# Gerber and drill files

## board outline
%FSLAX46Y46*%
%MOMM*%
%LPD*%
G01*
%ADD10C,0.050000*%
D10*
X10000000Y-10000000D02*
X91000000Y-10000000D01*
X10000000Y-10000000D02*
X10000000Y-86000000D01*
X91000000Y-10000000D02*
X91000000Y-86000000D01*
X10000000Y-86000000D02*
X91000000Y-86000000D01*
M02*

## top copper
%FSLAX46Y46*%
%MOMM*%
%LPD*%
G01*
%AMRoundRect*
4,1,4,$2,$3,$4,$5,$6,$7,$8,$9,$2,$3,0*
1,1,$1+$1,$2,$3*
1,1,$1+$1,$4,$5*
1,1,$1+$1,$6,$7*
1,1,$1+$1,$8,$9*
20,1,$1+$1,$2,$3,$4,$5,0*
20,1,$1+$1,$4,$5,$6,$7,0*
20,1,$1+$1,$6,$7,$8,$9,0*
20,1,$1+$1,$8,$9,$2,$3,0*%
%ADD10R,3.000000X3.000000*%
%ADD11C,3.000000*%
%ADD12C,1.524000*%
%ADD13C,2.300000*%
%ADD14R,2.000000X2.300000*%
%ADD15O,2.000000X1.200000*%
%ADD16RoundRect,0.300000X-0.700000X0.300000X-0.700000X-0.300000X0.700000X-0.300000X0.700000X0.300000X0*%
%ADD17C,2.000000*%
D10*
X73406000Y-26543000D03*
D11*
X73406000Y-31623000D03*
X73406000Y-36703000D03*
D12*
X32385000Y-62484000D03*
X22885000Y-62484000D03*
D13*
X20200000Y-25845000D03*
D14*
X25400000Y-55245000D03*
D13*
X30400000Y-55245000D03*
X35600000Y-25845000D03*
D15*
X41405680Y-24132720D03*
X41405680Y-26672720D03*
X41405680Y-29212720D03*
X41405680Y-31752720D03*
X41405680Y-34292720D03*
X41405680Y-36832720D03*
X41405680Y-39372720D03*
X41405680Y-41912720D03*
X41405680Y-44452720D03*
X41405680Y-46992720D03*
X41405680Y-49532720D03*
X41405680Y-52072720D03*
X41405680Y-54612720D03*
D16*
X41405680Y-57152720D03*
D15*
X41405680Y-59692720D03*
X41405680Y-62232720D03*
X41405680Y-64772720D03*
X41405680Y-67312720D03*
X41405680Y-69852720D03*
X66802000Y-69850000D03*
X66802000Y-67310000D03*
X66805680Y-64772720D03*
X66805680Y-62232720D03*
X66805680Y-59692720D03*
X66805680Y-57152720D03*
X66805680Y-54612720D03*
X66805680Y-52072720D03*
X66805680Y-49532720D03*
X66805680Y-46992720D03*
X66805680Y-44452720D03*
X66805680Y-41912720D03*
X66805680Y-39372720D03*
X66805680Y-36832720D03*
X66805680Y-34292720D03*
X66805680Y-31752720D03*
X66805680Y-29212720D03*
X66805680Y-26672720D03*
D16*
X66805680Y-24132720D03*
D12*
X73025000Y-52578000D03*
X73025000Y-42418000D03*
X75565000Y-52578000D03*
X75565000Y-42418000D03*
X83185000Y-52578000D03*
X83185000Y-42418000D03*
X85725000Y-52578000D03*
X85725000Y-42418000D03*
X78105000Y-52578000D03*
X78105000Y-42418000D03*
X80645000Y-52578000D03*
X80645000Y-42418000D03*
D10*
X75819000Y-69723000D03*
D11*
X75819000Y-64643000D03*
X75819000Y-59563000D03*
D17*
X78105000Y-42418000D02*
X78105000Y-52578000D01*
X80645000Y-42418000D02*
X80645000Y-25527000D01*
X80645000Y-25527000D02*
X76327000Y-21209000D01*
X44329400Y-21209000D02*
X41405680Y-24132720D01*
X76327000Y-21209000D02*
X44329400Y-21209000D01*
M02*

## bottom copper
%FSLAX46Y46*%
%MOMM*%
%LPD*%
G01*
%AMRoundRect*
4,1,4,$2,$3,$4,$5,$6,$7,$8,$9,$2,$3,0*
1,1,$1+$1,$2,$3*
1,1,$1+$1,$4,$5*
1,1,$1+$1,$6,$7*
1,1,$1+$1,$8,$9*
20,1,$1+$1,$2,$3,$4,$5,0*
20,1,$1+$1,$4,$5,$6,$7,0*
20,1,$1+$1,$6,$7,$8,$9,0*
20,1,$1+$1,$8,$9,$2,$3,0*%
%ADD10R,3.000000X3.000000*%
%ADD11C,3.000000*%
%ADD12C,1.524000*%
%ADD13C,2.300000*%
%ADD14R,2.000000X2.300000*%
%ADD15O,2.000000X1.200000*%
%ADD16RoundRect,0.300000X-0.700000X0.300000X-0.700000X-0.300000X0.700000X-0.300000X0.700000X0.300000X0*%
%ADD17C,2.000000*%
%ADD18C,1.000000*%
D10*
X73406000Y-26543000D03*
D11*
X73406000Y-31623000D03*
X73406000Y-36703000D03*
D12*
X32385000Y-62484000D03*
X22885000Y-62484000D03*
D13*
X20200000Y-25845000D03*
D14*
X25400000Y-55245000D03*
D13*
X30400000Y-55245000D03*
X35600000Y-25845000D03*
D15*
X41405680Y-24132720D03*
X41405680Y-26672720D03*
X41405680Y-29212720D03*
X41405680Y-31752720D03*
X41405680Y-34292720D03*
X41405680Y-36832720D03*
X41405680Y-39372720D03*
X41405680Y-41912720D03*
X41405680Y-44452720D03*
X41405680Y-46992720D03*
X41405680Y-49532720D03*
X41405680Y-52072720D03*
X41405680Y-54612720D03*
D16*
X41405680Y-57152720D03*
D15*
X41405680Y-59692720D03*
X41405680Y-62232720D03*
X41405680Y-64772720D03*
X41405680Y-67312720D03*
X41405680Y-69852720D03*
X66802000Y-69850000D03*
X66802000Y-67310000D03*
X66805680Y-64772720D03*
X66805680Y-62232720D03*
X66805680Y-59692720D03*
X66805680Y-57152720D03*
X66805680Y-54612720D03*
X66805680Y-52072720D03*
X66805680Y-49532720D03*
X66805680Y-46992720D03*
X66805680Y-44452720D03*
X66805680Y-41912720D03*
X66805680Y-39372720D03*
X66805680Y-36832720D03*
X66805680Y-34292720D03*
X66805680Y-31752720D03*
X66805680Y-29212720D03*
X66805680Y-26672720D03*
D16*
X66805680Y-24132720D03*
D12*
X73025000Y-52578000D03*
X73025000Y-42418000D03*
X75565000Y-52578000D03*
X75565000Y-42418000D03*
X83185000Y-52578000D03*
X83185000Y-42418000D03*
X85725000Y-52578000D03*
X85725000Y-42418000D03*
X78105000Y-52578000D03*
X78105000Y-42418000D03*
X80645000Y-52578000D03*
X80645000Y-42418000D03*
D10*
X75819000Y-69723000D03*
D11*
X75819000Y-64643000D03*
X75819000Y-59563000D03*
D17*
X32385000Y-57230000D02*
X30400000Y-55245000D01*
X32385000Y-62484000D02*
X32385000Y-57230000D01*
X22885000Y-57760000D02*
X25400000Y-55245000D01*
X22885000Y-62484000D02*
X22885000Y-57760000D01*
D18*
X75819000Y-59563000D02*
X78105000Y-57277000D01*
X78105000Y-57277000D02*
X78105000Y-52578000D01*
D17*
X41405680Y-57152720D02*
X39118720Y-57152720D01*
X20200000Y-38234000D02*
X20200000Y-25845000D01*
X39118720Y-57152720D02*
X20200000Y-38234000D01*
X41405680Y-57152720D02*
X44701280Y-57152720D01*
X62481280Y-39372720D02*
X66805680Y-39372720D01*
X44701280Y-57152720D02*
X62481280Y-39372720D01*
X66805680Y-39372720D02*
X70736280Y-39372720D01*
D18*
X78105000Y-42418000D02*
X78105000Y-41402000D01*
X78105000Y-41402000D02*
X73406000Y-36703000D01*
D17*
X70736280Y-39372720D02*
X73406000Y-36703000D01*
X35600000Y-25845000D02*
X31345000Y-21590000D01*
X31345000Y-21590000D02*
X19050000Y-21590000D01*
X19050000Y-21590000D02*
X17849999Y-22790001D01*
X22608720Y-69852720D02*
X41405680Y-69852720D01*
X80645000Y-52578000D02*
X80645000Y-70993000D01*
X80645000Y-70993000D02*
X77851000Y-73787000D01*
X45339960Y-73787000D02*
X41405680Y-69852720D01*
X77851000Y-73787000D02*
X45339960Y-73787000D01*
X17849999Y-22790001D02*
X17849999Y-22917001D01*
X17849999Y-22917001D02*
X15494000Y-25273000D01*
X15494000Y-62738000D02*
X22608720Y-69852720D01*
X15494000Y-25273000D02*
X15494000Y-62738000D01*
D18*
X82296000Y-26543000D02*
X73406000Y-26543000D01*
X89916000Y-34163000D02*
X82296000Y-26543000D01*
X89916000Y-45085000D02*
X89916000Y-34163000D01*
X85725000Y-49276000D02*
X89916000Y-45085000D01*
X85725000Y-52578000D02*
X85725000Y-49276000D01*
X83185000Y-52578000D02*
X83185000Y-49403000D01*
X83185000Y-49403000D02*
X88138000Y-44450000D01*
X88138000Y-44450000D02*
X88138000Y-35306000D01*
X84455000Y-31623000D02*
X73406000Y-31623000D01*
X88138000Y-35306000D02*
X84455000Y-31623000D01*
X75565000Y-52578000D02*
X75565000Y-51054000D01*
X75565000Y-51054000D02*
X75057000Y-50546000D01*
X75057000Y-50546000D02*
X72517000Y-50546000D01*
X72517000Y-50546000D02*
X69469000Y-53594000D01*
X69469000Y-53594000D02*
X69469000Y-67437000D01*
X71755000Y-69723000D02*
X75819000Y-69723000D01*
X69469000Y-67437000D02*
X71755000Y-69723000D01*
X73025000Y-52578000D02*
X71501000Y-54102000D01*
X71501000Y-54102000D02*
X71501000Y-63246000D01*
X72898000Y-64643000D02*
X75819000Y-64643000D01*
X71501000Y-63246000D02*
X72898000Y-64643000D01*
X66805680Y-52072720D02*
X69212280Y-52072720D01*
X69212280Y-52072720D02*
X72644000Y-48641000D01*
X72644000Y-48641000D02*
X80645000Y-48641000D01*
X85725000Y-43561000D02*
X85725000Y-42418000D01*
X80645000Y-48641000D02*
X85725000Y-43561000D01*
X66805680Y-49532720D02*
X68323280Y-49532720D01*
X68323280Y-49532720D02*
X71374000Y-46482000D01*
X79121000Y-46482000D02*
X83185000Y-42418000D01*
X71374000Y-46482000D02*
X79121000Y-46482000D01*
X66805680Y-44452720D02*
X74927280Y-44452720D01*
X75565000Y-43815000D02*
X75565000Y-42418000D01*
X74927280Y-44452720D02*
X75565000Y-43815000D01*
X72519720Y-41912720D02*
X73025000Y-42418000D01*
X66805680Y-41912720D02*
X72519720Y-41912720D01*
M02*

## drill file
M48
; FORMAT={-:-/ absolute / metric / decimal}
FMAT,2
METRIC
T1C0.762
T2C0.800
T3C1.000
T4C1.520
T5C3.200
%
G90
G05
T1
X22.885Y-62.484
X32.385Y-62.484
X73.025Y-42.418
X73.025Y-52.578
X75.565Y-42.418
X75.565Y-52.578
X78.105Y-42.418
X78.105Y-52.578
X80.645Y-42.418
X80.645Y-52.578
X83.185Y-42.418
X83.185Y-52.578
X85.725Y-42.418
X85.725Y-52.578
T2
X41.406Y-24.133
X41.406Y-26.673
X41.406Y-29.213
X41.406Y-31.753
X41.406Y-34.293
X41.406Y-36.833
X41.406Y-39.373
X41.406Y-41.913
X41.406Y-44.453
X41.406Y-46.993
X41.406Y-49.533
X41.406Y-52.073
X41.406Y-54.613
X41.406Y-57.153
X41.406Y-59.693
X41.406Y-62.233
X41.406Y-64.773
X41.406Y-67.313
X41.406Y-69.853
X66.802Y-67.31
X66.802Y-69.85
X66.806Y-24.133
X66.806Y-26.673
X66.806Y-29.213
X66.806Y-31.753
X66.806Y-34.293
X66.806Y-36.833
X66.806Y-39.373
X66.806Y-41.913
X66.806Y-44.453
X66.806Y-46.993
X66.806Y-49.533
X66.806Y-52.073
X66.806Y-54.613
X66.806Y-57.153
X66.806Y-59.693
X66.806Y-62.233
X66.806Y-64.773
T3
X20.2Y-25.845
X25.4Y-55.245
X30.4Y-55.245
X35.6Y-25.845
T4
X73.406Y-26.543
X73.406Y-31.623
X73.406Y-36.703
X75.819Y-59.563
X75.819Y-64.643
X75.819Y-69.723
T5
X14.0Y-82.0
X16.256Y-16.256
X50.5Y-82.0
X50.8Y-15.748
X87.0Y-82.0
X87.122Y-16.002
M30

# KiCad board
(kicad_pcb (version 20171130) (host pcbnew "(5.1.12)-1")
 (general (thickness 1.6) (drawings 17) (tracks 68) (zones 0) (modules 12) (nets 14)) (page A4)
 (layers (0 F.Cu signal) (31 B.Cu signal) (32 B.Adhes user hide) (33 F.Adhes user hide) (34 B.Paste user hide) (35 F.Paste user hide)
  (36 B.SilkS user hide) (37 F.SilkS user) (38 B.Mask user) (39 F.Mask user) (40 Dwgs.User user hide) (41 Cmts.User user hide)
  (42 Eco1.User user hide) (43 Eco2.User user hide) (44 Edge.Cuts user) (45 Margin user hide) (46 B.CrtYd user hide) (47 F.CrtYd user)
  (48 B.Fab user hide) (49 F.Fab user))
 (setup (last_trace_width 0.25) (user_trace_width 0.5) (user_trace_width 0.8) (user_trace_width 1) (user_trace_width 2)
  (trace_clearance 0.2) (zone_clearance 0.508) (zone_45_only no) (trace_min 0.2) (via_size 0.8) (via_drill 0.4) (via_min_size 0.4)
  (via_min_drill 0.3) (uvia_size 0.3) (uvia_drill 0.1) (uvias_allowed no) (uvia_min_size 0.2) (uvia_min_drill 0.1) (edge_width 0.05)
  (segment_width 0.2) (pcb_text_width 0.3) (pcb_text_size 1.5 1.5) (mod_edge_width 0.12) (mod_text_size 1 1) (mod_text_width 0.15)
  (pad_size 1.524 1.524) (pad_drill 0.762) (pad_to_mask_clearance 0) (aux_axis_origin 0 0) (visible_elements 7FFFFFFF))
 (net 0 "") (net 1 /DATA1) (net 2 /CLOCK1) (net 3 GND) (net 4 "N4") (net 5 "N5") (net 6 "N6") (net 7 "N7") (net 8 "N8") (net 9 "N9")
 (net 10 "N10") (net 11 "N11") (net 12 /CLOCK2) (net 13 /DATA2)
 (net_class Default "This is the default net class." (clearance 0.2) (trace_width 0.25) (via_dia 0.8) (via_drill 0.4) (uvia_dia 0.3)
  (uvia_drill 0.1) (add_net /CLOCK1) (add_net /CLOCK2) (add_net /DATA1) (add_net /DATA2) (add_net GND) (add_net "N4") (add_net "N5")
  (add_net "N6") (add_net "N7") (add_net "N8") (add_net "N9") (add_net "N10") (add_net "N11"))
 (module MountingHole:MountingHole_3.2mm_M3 (layer F.Cu) (at 87.122 16.002)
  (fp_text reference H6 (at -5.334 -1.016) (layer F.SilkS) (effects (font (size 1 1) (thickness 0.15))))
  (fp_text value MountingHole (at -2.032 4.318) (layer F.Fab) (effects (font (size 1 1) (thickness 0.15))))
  (pad 1 np_thru_hole circle (at 0 0) (size 3.2 3.2) (drill 3.2) (layers *.Cu *.Mask)))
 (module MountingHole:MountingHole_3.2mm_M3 (layer F.Cu) (at 50.8 15.748)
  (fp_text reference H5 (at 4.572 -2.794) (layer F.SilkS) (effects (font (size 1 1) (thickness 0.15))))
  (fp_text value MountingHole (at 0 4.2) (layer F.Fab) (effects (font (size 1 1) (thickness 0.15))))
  (pad 1 np_thru_hole circle (at 0 0) (size 3.2 3.2) (drill 3.2) (layers *.Cu *.Mask)))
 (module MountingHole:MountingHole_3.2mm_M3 (layer F.Cu) (at 16.256 16.256)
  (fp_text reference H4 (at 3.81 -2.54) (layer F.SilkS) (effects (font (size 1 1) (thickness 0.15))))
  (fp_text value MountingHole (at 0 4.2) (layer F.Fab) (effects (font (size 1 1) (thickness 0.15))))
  (pad 1 np_thru_hole circle (at 0 0) (size 3.2 3.2) (drill 3.2) (layers *.Cu *.Mask)))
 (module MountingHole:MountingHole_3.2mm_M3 (layer F.Cu) (at 14 82)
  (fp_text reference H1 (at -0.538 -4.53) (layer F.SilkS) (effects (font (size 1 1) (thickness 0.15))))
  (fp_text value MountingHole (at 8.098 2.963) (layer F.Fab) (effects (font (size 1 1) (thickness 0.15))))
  (pad 1 np_thru_hole circle (at 0 0) (size 3.2 3.2) (drill 3.2) (layers *.Cu *.Mask)))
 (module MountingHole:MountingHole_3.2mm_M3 (layer F.Cu) (at 50.5 82)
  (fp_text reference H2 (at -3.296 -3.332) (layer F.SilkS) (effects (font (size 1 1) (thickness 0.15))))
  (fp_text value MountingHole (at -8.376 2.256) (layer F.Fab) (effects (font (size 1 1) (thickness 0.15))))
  (pad 1 np_thru_hole circle (at 0 0) (size 3.2 3.2) (drill 3.2) (layers *.Cu *.Mask)))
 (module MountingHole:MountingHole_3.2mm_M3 (layer F.Cu) (at 87 82)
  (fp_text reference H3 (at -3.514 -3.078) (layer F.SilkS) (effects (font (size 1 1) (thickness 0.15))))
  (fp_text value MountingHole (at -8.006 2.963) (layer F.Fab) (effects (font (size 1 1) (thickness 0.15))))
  (pad 1 np_thru_hole circle (at 0 0) (size 3.2 3.2) (drill 3.2) (layers *.Cu *.Mask)))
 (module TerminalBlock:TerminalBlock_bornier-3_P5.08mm (layer F.Cu) (at 73.406 26.543 270)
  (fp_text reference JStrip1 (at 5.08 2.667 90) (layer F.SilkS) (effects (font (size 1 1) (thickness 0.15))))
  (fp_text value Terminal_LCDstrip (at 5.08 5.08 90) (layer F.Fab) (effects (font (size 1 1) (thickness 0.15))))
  (pad 1 thru_hole rect (at 0 0 270) (size 3 3) (drill 1.52) (layers *.Cu *.Mask) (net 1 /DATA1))
  (pad 2 thru_hole circle (at 5.08 0 270) (size 3 3) (drill 1.52) (layers *.Cu *.Mask) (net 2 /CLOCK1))
  (pad 3 thru_hole circle (at 10.16 0 270) (size 3 3) (drill 1.52) (layers *.Cu *.Mask) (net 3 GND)))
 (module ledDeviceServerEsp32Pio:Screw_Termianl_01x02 (layer F.Cu) (at 37.719 60.452 270)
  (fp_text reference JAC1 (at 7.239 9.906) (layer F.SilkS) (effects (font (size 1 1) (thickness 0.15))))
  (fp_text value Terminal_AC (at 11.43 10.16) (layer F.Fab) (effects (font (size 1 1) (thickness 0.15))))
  (pad 1 thru_hole circle (at 2.032 5.334 270) (size 1.524 1.524) (drill 0.762) (layers *.Cu *.Mask) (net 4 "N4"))
  (pad 2 thru_hole circle (at 2.032 14.834 270) (size 1.524 1.524) (drill 0.762) (layers *.Cu *.Mask) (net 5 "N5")))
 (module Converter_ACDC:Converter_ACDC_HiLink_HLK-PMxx (layer F.Cu) (at 25.4 55.245 90)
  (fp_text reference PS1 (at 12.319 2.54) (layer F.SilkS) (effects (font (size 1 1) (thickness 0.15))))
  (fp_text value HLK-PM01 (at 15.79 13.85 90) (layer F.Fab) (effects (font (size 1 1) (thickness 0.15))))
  (pad 3 thru_hole circle (at 29.4 -5.2 90) (size 2.3 2.3) (drill 1) (layers *.Cu *.Mask) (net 3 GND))
  (pad 1 thru_hole rect (at 0 0 90) (size 2.3 2) (drill 1) (layers *.Cu *.Mask) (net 5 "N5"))
  (pad 2 thru_hole circle (at 0 5 90) (size 2.3 2.3) (drill 1) (layers *.Cu *.Mask) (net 4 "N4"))
  (pad 4 thru_hole circle (at 29.4 10.2 90) (size 2.3 2.3) (drill 1) (layers *.Cu *.Mask) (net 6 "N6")))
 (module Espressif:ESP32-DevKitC (layer F.Cu) (at 41.402 24.13)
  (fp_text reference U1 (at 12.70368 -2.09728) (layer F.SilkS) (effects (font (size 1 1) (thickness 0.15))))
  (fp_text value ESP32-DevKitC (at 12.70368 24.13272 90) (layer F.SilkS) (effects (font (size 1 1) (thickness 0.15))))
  (pad 1 thru_hole oval (at 0.00368 0.00272 270) (size 1.2 2) (drill 0.8) (layers *.Cu *.Mask) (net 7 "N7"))
  (pad 2 thru_hole oval (at 0.00368 2.54272 270) (size 1.2 2) (drill 0.8) (layers *.Cu *.Mask))
  (pad 3 thru_hole oval (at 0.00368 5.08272 270) (size 1.2 2) (drill 0.8) (layers *.Cu *.Mask))
  (pad 4 thru_hole oval (at 0.00368 7.62272 270) (size 1.2 2) (drill 0.8) (layers *.Cu *.Mask))
  (pad 5 thru_hole oval (at 0.00368 10.16272 270) (size 1.2 2) (drill 0.8) (layers *.Cu *.Mask))
  (pad 6 thru_hole oval (at 0.00368 12.70272 270) (size 1.2 2) (drill 0.8) (layers *.Cu *.Mask))
  (pad 7 thru_hole oval (at 0.00368 15.24272 270) (size 1.2 2) (drill 0.8) (layers *.Cu *.Mask))
  (pad 8 thru_hole oval (at 0.00368 17.78272 270) (size 1.2 2) (drill 0.8) (layers *.Cu *.Mask))
  (pad 9 thru_hole oval (at 0.00368 20.32272 270) (size 1.2 2) (drill 0.8) (layers *.Cu *.Mask))
  (pad 10 thru_hole oval (at 0.00368 22.86272 270) (size 1.2 2) (drill 0.8) (layers *.Cu *.Mask))
  (pad 11 thru_hole oval (at 0.00368 25.40272 270) (size 1.2 2) (drill 0.8) (layers *.Cu *.Mask))
  (pad 12 thru_hole oval (at 0.00368 27.94272 270) (size 1.2 2) (drill 0.8) (layers *.Cu *.Mask))
  (pad 13 thru_hole oval (at 0.00368 30.48272 270) (size 1.2 2) (drill 0.8) (layers *.Cu *.Mask))
  (pad 14 thru_hole roundrect (at 0.00368 33.02272 270) (size 1.2 2) (drill 0.8) (layers *.Cu *.Mask) (roundrect_rratio 0.25) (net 3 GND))
  (pad 15 thru_hole oval (at 0.00368 35.56272 270) (size 1.2 2) (drill 0.8) (layers *.Cu *.Mask))
  (pad 16 thru_hole oval (at 0.00368 38.10272 270) (size 1.2 2) (drill 0.8) (layers *.Cu *.Mask))
  (pad 17 thru_hole oval (at 0.00368 40.64272 270) (size 1.2 2) (drill 0.8) (layers *.Cu *.Mask))
  (pad 18 thru_hole oval (at 0.00368 43.18272 270) (size 1.2 2) (drill 0.8) (layers *.Cu *.Mask))
  (pad 19 thru_hole oval (at 0.00368 45.72272 270) (size 1.2 2) (drill 0.8) (layers *.Cu *.Mask) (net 6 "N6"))
  (pad 20 thru_hole oval (at 25.4 45.72 270) (size 1.2 2) (drill 0.8) (layers *.Cu *.Mask))
  (pad 21 thru_hole oval (at 25.4 43.18 270) (size 1.2 2) (drill 0.8) (layers *.Cu *.Mask))
  (pad 22 thru_hole oval (at 25.40368 40.64272 270) (size 1.2 2) (drill 0.8) (layers *.Cu *.Mask))
  (pad 23 thru_hole oval (at 25.40368 38.10272 270) (size 1.2 2) (drill 0.8) (layers *.Cu *.Mask))
  (pad 24 thru_hole oval (at 25.40368 35.56272 270) (size 1.2 2) (drill 0.8) (layers *.Cu *.Mask))
  (pad 25 thru_hole oval (at 25.40368 33.02272 270) (size 1.2 2) (drill 0.8) (layers *.Cu *.Mask))
  (pad 26 thru_hole oval (at 25.40368 30.48272 270) (size 1.2 2) (drill 0.8) (layers *.Cu *.Mask))
  (pad 27 thru_hole oval (at 25.40368 27.94272 270) (size 1.2 2) (drill 0.8) (layers *.Cu *.Mask) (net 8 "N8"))
  (pad 28 thru_hole oval (at 25.40368 25.40272 270) (size 1.2 2) (drill 0.8) (layers *.Cu *.Mask) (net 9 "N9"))
  (pad 29 thru_hole oval (at 25.40368 22.86272 270) (size 1.2 2) (drill 0.8) (layers *.Cu *.Mask))
  (pad 30 thru_hole oval (at 25.40368 20.32272 270) (size 1.2 2) (drill 0.8) (layers *.Cu *.Mask) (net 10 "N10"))
  (pad 31 thru_hole oval (at 25.40368 17.78272 270) (size 1.2 2) (drill 0.8) (layers *.Cu *.Mask) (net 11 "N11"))
  (pad 32 thru_hole oval (at 25.40368 15.24272 270) (size 1.2 2) (drill 0.8) (layers *.Cu *.Mask) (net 3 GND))
  (pad 33 thru_hole oval (at 25.40368 12.70272 270) (size 1.2 2) (drill 0.8) (layers *.Cu *.Mask))
  (pad 34 thru_hole oval (at 25.40368 10.16272 270) (size 1.2 2) (drill 0.8) (layers *.Cu *.Mask))
  (pad 35 thru_hole oval (at 25.40368 7.62272 270) (size 1.2 2) (drill 0.8) (layers *.Cu *.Mask))
  (pad 36 thru_hole oval (at 25.40368 5.08272 270) (size 1.2 2) (drill 0.8) (layers *.Cu *.Mask))
  (pad 37 thru_hole oval (at 25.40368 2.54272 270) (size 1.2 2) (drill 0.8) (layers *.Cu *.Mask))
  (pad 38 thru_hole roundrect (at 25.40368 0.00272 270) (size 1.2 2) (drill 0.8) (layers *.Cu *.Mask) (roundrect_rratio 0.25)))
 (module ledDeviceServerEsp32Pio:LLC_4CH (layer F.Cu) (at 87.122 53.975 180)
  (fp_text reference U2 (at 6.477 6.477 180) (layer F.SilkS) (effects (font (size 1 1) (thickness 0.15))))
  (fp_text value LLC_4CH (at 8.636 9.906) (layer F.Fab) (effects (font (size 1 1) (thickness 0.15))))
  (pad 11 thru_hole circle (at 14.097 1.397 180) (size 1.524 1.524) (drill 0.762) (layers *.Cu *.Mask) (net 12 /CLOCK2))
  (pad 10 thru_hole circle (at 14.097 11.557 180) (size 1.524 1.524) (drill 0.762) (layers *.Cu *.Mask) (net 11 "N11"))
  (pad 9 thru_hole circle (at 11.557 1.397 180) (size 1.524 1.524) (drill 0.762) (layers *.Cu *.Mask) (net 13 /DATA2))
  (pad 8 thru_hole circle (at 11.557 11.557 180) (size 1.524 1.524) (drill 0.762) (layers *.Cu *.Mask) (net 10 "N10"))
  (pad 7 thru_hole circle (at 3.937 1.397 180) (size 1.524 1.524) (drill 0.762) (layers *.Cu *.Mask) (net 2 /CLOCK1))
  (pad 6 thru_hole circle (at 3.937 11.557 180) (size 1.524 1.524) (drill 0.762) (layers *.Cu *.Mask) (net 9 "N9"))
  (pad 5 thru_hole circle (at 1.397 1.397 180) (size 1.524 1.524) (drill 0.762) (layers *.Cu *.Mask) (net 1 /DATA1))
  (pad 4 thru_hole circle (at 1.397 11.557 180) (size 1.524 1.524) (drill 0.762) (layers *.Cu *.Mask) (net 8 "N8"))
  (pad 3 thru_hole circle (at 9.017 1.397 180) (size 1.524 1.524) (drill 0.762) (layers *.Cu *.Mask) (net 3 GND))
  (pad 3 thru_hole circle (at 9.017 11.557 180) (size 1.524 1.524) (drill 0.762) (layers *.Cu *.Mask) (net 3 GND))
  (pad 2 thru_hole circle (at 6.477 1.397 180) (size 1.524 1.524) (drill 0.762) (layers *.Cu *.Mask) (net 6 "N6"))
  (pad 1 thru_hole circle (at 6.477 11.557 180) (size 1.524 1.524) (drill 0.762) (layers *.Cu *.Mask) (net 7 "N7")))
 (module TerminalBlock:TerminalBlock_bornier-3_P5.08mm (layer F.Cu) (at 75.819 69.723 90)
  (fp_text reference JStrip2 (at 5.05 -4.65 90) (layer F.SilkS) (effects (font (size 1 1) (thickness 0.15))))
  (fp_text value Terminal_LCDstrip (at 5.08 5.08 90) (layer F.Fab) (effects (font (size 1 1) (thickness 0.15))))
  (pad 1 thru_hole rect (at 0 0 90) (size 3 3) (drill 1.52) (layers *.Cu *.Mask) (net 13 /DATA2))
  (pad 2 thru_hole circle (at 5.08 0 90) (size 3 3) (drill 1.52) (layers *.Cu *.Mask) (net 12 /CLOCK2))
  (pad 3 thru_hole circle (at 10.16 0 90) (size 3 3) (drill 1.52) (layers *.Cu *.Mask) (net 3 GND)))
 (gr_line (start 10 10) (end 91 10) (layer Edge.Cuts) (width 0.05))
 (gr_line (start 10 10) (end 10 86) (layer Edge.Cuts) (width 0.05))
 (gr_line (start 91 10) (end 91 86) (layer Edge.Cuts) (width 0.05))
 (gr_line (start 10 86) (end 91 86) (layer Edge.Cuts) (width 0.05))
 (segment (start 32.385 57.23) (end 30.4 55.245) (width 2) (layer B.Cu) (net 4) (status 20))
 (segment (start 32.385 62.484) (end 32.385 57.23) (width 2) (layer B.Cu) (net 4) (status 10))
 (segment (start 22.885 57.76) (end 25.4 55.245) (width 2) (layer B.Cu) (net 5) (status 20))
 (segment (start 22.885 62.484) (end 22.885 57.76) (width 2) (layer B.Cu) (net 5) (status 10))
 (segment (start 75.819 59.563) (end 78.105 57.277) (width 1) (layer B.Cu) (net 3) (status 10))
 (segment (start 78.105 57.277) (end 78.105 52.578) (width 1) (layer B.Cu) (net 3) (status 20))
 (segment (start 41.40568 57.15272) (end 39.11872 57.15272) (width 2) (layer B.Cu) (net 3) (status 10))
 (segment (start 20.2 38.234) (end 20.2 25.845) (width 2) (layer B.Cu) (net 3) (status 20))
 (segment (start 39.11872 57.15272) (end 20.2 38.234) (width 2) (layer B.Cu) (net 3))
 (segment (start 41.40568 57.15272) (end 44.70128 57.15272) (width 2) (layer B.Cu) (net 3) (status 10))
 (segment (start 62.48128 39.37272) (end 66.80568 39.37272) (width 2) (layer B.Cu) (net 3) (status 20))
 (segment (start 44.70128 57.15272) (end 62.48128 39.37272) (width 2) (layer B.Cu) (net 3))
 (segment (start 66.80568 39.37272) (end 70.73628 39.37272) (width 2) (layer B.Cu) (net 3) (status 10))
 (segment (start 78.105 42.418) (end 78.105 52.578) (width 2) (layer F.Cu) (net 3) (status 30))
 (segment (start 78.105 42.418) (end 78.105 41.402) (width 1) (layer B.Cu) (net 3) (status 10))
 (segment (start 78.105 41.402) (end 73.406 36.703) (width 1) (layer B.Cu) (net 3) (status 20))
 (segment (start 70.73628 39.37272) (end 73.406 36.703) (width 2) (layer B.Cu) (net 3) (status 20))
 (segment (start 35.6 25.845) (end 31.345 21.59) (width 2) (layer B.Cu) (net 6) (status 10))
 (segment (start 31.345 21.59) (end 19.05 21.59) (width 2) (layer B.Cu) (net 6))
 (segment (start 19.05 21.59) (end 17.849999 22.790001) (width 2) (layer B.Cu) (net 6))
 (segment (start 22.60872 69.85272) (end 41.40568 69.85272) (width 2) (layer B.Cu) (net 6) (status 20))
 (segment (start 80.645 52.578) (end 80.645 70.993) (width 2) (layer B.Cu) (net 6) (status 10))
 (segment (start 80.645 70.993) (end 77.851 73.787) (width 2) (layer B.Cu) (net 6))
 (segment (start 45.33996 73.787) (end 41.40568 69.85272) (width 2) (layer B.Cu) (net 6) (status 20))
 (segment (start 77.851 73.787) (end 45.33996 73.787) (width 2) (layer B.Cu) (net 6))
 (segment (start 17.849999 22.790001) (end 17.849999 22.917001) (width 2) (layer B.Cu) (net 6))
 (segment (start 17.849999 22.917001) (end 15.494 25.273) (width 2) (layer B.Cu) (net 6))
 (segment (start 15.494 62.738) (end 22.60872 69.85272) (width 2) (layer B.Cu) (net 6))
 (segment (start 15.494 25.273) (end 15.494 62.738) (width 2) (layer B.Cu) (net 6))
 (segment (start 82.296 26.543) (end 73.406 26.543) (width 1) (layer B.Cu) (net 1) (status 20))
 (segment (start 89.916 34.163) (end 82.296 26.543) (width 1) (layer B.Cu) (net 1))
 (segment (start 89.916 45.085) (end 89.916 34.163) (width 1) (layer B.Cu) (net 1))
 (segment (start 85.725 49.276) (end 89.916 45.085) (width 1) (layer B.Cu) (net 1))
 (segment (start 85.725 52.578) (end 85.725 49.276) (width 1) (layer B.Cu) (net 1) (status 10))
 (segment (start 83.185 52.578) (end 83.185 49.403) (width 1) (layer B.Cu) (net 2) (status 10))
 (segment (start 83.185 49.403) (end 88.138 44.45) (width 1) (layer B.Cu) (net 2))
 (segment (start 88.138 44.45) (end 88.138 35.306) (width 1) (layer B.Cu) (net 2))
 (segment (start 84.455 31.623) (end 73.406 31.623) (width 1) (layer B.Cu) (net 2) (status 20))
 (segment (start 88.138 35.306) (end 84.455 31.623) (width 1) (layer B.Cu) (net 2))
 (segment (start 75.565 52.578) (end 75.565 51.054) (width 1) (layer B.Cu) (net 13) (status 10))
 (segment (start 75.565 51.054) (end 75.057 50.546) (width 1) (layer B.Cu) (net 13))
 (segment (start 75.057 50.546) (end 72.517 50.546) (width 1) (layer B.Cu) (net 13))
 (segment (start 72.517 50.546) (end 69.469 53.594) (width 1) (layer B.Cu) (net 13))
 (segment (start 69.469 53.594) (end 69.469 67.437) (width 1) (layer B.Cu) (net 13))
 (segment (start 71.755 69.723) (end 75.819 69.723) (width 1) (layer B.Cu) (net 13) (status 20))
 (segment (start 69.469 67.437) (end 71.755 69.723) (width 1) (layer B.Cu) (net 13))
 (segment (start 73.025 52.578) (end 71.501 54.102) (width 1) (layer B.Cu) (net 12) (status 10))
 (segment (start 71.501 54.102) (end 71.501 63.246) (width 1) (layer B.Cu) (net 12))
 (segment (start 72.898 64.643) (end 75.819 64.643) (width 1) (layer B.Cu) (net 12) (status 20))
 (segment (start 71.501 63.246) (end 72.898 64.643) (width 1) (layer B.Cu) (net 12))
 (segment (start 80.645 42.418) (end 80.645 25.527) (width 2) (layer F.Cu) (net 7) (status 10))
 (segment (start 80.645 25.527) (end 76.327 21.209) (width 2) (layer F.Cu) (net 7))
 (segment (start 44.3294 21.209) (end 41.40568 24.13272) (width 2) (layer F.Cu) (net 7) (status 20))
 (segment (start 76.327 21.209) (end 44.3294 21.209) (width 2) (layer F.Cu) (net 7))
 (segment (start 66.80568 52.07272) (end 69.21228 52.07272) (width 1) (layer B.Cu) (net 8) (status 10))
 (segment (start 69.21228 52.07272) (end 72.644 48.641) (width 1) (layer B.Cu) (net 8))
 (segment (start 72.644 48.641) (end 80.645 48.641) (width 1) (layer B.Cu) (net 8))
 (segment (start 85.725 43.561) (end 85.725 42.418) (width 1) (layer B.Cu) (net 8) (status 20))
 (segment (start 80.645 48.641) (end 85.725 43.561) (width 1) (layer B.Cu) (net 8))
 (segment (start 66.80568 49.53272) (end 68.32328 49.53272) (width 1) (layer B.Cu) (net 9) (status 10))
 (segment (start 68.32328 49.53272) (end 71.374 46.482) (width 1) (layer B.Cu) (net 9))
 (segment (start 79.121 46.482) (end 83.185 42.418) (width 1) (layer B.Cu) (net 9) (status 20))
 (segment (start 71.374 46.482) (end 79.121 46.482) (width 1) (layer B.Cu) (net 9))
 (segment (start 66.80568 44.45272) (end 74.92728 44.45272) (width 1) (layer B.Cu) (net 10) (status 10))
 (segment (start 75.565 43.815) (end 75.565 42.418) (width 1) (layer B.Cu) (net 10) (status 20))
 (segment (start 74.92728 44.45272) (end 75.565 43.815) (width 1) (layer B.Cu) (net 10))
 (segment (start 72.51972 41.91272) (end 73.025 42.418) (width 1) (layer B.Cu) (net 11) (status 30))
 (segment (start 66.80568 41.91272) (end 72.51972 41.91272) (width 1) (layer B.Cu) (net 11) (status 30)))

